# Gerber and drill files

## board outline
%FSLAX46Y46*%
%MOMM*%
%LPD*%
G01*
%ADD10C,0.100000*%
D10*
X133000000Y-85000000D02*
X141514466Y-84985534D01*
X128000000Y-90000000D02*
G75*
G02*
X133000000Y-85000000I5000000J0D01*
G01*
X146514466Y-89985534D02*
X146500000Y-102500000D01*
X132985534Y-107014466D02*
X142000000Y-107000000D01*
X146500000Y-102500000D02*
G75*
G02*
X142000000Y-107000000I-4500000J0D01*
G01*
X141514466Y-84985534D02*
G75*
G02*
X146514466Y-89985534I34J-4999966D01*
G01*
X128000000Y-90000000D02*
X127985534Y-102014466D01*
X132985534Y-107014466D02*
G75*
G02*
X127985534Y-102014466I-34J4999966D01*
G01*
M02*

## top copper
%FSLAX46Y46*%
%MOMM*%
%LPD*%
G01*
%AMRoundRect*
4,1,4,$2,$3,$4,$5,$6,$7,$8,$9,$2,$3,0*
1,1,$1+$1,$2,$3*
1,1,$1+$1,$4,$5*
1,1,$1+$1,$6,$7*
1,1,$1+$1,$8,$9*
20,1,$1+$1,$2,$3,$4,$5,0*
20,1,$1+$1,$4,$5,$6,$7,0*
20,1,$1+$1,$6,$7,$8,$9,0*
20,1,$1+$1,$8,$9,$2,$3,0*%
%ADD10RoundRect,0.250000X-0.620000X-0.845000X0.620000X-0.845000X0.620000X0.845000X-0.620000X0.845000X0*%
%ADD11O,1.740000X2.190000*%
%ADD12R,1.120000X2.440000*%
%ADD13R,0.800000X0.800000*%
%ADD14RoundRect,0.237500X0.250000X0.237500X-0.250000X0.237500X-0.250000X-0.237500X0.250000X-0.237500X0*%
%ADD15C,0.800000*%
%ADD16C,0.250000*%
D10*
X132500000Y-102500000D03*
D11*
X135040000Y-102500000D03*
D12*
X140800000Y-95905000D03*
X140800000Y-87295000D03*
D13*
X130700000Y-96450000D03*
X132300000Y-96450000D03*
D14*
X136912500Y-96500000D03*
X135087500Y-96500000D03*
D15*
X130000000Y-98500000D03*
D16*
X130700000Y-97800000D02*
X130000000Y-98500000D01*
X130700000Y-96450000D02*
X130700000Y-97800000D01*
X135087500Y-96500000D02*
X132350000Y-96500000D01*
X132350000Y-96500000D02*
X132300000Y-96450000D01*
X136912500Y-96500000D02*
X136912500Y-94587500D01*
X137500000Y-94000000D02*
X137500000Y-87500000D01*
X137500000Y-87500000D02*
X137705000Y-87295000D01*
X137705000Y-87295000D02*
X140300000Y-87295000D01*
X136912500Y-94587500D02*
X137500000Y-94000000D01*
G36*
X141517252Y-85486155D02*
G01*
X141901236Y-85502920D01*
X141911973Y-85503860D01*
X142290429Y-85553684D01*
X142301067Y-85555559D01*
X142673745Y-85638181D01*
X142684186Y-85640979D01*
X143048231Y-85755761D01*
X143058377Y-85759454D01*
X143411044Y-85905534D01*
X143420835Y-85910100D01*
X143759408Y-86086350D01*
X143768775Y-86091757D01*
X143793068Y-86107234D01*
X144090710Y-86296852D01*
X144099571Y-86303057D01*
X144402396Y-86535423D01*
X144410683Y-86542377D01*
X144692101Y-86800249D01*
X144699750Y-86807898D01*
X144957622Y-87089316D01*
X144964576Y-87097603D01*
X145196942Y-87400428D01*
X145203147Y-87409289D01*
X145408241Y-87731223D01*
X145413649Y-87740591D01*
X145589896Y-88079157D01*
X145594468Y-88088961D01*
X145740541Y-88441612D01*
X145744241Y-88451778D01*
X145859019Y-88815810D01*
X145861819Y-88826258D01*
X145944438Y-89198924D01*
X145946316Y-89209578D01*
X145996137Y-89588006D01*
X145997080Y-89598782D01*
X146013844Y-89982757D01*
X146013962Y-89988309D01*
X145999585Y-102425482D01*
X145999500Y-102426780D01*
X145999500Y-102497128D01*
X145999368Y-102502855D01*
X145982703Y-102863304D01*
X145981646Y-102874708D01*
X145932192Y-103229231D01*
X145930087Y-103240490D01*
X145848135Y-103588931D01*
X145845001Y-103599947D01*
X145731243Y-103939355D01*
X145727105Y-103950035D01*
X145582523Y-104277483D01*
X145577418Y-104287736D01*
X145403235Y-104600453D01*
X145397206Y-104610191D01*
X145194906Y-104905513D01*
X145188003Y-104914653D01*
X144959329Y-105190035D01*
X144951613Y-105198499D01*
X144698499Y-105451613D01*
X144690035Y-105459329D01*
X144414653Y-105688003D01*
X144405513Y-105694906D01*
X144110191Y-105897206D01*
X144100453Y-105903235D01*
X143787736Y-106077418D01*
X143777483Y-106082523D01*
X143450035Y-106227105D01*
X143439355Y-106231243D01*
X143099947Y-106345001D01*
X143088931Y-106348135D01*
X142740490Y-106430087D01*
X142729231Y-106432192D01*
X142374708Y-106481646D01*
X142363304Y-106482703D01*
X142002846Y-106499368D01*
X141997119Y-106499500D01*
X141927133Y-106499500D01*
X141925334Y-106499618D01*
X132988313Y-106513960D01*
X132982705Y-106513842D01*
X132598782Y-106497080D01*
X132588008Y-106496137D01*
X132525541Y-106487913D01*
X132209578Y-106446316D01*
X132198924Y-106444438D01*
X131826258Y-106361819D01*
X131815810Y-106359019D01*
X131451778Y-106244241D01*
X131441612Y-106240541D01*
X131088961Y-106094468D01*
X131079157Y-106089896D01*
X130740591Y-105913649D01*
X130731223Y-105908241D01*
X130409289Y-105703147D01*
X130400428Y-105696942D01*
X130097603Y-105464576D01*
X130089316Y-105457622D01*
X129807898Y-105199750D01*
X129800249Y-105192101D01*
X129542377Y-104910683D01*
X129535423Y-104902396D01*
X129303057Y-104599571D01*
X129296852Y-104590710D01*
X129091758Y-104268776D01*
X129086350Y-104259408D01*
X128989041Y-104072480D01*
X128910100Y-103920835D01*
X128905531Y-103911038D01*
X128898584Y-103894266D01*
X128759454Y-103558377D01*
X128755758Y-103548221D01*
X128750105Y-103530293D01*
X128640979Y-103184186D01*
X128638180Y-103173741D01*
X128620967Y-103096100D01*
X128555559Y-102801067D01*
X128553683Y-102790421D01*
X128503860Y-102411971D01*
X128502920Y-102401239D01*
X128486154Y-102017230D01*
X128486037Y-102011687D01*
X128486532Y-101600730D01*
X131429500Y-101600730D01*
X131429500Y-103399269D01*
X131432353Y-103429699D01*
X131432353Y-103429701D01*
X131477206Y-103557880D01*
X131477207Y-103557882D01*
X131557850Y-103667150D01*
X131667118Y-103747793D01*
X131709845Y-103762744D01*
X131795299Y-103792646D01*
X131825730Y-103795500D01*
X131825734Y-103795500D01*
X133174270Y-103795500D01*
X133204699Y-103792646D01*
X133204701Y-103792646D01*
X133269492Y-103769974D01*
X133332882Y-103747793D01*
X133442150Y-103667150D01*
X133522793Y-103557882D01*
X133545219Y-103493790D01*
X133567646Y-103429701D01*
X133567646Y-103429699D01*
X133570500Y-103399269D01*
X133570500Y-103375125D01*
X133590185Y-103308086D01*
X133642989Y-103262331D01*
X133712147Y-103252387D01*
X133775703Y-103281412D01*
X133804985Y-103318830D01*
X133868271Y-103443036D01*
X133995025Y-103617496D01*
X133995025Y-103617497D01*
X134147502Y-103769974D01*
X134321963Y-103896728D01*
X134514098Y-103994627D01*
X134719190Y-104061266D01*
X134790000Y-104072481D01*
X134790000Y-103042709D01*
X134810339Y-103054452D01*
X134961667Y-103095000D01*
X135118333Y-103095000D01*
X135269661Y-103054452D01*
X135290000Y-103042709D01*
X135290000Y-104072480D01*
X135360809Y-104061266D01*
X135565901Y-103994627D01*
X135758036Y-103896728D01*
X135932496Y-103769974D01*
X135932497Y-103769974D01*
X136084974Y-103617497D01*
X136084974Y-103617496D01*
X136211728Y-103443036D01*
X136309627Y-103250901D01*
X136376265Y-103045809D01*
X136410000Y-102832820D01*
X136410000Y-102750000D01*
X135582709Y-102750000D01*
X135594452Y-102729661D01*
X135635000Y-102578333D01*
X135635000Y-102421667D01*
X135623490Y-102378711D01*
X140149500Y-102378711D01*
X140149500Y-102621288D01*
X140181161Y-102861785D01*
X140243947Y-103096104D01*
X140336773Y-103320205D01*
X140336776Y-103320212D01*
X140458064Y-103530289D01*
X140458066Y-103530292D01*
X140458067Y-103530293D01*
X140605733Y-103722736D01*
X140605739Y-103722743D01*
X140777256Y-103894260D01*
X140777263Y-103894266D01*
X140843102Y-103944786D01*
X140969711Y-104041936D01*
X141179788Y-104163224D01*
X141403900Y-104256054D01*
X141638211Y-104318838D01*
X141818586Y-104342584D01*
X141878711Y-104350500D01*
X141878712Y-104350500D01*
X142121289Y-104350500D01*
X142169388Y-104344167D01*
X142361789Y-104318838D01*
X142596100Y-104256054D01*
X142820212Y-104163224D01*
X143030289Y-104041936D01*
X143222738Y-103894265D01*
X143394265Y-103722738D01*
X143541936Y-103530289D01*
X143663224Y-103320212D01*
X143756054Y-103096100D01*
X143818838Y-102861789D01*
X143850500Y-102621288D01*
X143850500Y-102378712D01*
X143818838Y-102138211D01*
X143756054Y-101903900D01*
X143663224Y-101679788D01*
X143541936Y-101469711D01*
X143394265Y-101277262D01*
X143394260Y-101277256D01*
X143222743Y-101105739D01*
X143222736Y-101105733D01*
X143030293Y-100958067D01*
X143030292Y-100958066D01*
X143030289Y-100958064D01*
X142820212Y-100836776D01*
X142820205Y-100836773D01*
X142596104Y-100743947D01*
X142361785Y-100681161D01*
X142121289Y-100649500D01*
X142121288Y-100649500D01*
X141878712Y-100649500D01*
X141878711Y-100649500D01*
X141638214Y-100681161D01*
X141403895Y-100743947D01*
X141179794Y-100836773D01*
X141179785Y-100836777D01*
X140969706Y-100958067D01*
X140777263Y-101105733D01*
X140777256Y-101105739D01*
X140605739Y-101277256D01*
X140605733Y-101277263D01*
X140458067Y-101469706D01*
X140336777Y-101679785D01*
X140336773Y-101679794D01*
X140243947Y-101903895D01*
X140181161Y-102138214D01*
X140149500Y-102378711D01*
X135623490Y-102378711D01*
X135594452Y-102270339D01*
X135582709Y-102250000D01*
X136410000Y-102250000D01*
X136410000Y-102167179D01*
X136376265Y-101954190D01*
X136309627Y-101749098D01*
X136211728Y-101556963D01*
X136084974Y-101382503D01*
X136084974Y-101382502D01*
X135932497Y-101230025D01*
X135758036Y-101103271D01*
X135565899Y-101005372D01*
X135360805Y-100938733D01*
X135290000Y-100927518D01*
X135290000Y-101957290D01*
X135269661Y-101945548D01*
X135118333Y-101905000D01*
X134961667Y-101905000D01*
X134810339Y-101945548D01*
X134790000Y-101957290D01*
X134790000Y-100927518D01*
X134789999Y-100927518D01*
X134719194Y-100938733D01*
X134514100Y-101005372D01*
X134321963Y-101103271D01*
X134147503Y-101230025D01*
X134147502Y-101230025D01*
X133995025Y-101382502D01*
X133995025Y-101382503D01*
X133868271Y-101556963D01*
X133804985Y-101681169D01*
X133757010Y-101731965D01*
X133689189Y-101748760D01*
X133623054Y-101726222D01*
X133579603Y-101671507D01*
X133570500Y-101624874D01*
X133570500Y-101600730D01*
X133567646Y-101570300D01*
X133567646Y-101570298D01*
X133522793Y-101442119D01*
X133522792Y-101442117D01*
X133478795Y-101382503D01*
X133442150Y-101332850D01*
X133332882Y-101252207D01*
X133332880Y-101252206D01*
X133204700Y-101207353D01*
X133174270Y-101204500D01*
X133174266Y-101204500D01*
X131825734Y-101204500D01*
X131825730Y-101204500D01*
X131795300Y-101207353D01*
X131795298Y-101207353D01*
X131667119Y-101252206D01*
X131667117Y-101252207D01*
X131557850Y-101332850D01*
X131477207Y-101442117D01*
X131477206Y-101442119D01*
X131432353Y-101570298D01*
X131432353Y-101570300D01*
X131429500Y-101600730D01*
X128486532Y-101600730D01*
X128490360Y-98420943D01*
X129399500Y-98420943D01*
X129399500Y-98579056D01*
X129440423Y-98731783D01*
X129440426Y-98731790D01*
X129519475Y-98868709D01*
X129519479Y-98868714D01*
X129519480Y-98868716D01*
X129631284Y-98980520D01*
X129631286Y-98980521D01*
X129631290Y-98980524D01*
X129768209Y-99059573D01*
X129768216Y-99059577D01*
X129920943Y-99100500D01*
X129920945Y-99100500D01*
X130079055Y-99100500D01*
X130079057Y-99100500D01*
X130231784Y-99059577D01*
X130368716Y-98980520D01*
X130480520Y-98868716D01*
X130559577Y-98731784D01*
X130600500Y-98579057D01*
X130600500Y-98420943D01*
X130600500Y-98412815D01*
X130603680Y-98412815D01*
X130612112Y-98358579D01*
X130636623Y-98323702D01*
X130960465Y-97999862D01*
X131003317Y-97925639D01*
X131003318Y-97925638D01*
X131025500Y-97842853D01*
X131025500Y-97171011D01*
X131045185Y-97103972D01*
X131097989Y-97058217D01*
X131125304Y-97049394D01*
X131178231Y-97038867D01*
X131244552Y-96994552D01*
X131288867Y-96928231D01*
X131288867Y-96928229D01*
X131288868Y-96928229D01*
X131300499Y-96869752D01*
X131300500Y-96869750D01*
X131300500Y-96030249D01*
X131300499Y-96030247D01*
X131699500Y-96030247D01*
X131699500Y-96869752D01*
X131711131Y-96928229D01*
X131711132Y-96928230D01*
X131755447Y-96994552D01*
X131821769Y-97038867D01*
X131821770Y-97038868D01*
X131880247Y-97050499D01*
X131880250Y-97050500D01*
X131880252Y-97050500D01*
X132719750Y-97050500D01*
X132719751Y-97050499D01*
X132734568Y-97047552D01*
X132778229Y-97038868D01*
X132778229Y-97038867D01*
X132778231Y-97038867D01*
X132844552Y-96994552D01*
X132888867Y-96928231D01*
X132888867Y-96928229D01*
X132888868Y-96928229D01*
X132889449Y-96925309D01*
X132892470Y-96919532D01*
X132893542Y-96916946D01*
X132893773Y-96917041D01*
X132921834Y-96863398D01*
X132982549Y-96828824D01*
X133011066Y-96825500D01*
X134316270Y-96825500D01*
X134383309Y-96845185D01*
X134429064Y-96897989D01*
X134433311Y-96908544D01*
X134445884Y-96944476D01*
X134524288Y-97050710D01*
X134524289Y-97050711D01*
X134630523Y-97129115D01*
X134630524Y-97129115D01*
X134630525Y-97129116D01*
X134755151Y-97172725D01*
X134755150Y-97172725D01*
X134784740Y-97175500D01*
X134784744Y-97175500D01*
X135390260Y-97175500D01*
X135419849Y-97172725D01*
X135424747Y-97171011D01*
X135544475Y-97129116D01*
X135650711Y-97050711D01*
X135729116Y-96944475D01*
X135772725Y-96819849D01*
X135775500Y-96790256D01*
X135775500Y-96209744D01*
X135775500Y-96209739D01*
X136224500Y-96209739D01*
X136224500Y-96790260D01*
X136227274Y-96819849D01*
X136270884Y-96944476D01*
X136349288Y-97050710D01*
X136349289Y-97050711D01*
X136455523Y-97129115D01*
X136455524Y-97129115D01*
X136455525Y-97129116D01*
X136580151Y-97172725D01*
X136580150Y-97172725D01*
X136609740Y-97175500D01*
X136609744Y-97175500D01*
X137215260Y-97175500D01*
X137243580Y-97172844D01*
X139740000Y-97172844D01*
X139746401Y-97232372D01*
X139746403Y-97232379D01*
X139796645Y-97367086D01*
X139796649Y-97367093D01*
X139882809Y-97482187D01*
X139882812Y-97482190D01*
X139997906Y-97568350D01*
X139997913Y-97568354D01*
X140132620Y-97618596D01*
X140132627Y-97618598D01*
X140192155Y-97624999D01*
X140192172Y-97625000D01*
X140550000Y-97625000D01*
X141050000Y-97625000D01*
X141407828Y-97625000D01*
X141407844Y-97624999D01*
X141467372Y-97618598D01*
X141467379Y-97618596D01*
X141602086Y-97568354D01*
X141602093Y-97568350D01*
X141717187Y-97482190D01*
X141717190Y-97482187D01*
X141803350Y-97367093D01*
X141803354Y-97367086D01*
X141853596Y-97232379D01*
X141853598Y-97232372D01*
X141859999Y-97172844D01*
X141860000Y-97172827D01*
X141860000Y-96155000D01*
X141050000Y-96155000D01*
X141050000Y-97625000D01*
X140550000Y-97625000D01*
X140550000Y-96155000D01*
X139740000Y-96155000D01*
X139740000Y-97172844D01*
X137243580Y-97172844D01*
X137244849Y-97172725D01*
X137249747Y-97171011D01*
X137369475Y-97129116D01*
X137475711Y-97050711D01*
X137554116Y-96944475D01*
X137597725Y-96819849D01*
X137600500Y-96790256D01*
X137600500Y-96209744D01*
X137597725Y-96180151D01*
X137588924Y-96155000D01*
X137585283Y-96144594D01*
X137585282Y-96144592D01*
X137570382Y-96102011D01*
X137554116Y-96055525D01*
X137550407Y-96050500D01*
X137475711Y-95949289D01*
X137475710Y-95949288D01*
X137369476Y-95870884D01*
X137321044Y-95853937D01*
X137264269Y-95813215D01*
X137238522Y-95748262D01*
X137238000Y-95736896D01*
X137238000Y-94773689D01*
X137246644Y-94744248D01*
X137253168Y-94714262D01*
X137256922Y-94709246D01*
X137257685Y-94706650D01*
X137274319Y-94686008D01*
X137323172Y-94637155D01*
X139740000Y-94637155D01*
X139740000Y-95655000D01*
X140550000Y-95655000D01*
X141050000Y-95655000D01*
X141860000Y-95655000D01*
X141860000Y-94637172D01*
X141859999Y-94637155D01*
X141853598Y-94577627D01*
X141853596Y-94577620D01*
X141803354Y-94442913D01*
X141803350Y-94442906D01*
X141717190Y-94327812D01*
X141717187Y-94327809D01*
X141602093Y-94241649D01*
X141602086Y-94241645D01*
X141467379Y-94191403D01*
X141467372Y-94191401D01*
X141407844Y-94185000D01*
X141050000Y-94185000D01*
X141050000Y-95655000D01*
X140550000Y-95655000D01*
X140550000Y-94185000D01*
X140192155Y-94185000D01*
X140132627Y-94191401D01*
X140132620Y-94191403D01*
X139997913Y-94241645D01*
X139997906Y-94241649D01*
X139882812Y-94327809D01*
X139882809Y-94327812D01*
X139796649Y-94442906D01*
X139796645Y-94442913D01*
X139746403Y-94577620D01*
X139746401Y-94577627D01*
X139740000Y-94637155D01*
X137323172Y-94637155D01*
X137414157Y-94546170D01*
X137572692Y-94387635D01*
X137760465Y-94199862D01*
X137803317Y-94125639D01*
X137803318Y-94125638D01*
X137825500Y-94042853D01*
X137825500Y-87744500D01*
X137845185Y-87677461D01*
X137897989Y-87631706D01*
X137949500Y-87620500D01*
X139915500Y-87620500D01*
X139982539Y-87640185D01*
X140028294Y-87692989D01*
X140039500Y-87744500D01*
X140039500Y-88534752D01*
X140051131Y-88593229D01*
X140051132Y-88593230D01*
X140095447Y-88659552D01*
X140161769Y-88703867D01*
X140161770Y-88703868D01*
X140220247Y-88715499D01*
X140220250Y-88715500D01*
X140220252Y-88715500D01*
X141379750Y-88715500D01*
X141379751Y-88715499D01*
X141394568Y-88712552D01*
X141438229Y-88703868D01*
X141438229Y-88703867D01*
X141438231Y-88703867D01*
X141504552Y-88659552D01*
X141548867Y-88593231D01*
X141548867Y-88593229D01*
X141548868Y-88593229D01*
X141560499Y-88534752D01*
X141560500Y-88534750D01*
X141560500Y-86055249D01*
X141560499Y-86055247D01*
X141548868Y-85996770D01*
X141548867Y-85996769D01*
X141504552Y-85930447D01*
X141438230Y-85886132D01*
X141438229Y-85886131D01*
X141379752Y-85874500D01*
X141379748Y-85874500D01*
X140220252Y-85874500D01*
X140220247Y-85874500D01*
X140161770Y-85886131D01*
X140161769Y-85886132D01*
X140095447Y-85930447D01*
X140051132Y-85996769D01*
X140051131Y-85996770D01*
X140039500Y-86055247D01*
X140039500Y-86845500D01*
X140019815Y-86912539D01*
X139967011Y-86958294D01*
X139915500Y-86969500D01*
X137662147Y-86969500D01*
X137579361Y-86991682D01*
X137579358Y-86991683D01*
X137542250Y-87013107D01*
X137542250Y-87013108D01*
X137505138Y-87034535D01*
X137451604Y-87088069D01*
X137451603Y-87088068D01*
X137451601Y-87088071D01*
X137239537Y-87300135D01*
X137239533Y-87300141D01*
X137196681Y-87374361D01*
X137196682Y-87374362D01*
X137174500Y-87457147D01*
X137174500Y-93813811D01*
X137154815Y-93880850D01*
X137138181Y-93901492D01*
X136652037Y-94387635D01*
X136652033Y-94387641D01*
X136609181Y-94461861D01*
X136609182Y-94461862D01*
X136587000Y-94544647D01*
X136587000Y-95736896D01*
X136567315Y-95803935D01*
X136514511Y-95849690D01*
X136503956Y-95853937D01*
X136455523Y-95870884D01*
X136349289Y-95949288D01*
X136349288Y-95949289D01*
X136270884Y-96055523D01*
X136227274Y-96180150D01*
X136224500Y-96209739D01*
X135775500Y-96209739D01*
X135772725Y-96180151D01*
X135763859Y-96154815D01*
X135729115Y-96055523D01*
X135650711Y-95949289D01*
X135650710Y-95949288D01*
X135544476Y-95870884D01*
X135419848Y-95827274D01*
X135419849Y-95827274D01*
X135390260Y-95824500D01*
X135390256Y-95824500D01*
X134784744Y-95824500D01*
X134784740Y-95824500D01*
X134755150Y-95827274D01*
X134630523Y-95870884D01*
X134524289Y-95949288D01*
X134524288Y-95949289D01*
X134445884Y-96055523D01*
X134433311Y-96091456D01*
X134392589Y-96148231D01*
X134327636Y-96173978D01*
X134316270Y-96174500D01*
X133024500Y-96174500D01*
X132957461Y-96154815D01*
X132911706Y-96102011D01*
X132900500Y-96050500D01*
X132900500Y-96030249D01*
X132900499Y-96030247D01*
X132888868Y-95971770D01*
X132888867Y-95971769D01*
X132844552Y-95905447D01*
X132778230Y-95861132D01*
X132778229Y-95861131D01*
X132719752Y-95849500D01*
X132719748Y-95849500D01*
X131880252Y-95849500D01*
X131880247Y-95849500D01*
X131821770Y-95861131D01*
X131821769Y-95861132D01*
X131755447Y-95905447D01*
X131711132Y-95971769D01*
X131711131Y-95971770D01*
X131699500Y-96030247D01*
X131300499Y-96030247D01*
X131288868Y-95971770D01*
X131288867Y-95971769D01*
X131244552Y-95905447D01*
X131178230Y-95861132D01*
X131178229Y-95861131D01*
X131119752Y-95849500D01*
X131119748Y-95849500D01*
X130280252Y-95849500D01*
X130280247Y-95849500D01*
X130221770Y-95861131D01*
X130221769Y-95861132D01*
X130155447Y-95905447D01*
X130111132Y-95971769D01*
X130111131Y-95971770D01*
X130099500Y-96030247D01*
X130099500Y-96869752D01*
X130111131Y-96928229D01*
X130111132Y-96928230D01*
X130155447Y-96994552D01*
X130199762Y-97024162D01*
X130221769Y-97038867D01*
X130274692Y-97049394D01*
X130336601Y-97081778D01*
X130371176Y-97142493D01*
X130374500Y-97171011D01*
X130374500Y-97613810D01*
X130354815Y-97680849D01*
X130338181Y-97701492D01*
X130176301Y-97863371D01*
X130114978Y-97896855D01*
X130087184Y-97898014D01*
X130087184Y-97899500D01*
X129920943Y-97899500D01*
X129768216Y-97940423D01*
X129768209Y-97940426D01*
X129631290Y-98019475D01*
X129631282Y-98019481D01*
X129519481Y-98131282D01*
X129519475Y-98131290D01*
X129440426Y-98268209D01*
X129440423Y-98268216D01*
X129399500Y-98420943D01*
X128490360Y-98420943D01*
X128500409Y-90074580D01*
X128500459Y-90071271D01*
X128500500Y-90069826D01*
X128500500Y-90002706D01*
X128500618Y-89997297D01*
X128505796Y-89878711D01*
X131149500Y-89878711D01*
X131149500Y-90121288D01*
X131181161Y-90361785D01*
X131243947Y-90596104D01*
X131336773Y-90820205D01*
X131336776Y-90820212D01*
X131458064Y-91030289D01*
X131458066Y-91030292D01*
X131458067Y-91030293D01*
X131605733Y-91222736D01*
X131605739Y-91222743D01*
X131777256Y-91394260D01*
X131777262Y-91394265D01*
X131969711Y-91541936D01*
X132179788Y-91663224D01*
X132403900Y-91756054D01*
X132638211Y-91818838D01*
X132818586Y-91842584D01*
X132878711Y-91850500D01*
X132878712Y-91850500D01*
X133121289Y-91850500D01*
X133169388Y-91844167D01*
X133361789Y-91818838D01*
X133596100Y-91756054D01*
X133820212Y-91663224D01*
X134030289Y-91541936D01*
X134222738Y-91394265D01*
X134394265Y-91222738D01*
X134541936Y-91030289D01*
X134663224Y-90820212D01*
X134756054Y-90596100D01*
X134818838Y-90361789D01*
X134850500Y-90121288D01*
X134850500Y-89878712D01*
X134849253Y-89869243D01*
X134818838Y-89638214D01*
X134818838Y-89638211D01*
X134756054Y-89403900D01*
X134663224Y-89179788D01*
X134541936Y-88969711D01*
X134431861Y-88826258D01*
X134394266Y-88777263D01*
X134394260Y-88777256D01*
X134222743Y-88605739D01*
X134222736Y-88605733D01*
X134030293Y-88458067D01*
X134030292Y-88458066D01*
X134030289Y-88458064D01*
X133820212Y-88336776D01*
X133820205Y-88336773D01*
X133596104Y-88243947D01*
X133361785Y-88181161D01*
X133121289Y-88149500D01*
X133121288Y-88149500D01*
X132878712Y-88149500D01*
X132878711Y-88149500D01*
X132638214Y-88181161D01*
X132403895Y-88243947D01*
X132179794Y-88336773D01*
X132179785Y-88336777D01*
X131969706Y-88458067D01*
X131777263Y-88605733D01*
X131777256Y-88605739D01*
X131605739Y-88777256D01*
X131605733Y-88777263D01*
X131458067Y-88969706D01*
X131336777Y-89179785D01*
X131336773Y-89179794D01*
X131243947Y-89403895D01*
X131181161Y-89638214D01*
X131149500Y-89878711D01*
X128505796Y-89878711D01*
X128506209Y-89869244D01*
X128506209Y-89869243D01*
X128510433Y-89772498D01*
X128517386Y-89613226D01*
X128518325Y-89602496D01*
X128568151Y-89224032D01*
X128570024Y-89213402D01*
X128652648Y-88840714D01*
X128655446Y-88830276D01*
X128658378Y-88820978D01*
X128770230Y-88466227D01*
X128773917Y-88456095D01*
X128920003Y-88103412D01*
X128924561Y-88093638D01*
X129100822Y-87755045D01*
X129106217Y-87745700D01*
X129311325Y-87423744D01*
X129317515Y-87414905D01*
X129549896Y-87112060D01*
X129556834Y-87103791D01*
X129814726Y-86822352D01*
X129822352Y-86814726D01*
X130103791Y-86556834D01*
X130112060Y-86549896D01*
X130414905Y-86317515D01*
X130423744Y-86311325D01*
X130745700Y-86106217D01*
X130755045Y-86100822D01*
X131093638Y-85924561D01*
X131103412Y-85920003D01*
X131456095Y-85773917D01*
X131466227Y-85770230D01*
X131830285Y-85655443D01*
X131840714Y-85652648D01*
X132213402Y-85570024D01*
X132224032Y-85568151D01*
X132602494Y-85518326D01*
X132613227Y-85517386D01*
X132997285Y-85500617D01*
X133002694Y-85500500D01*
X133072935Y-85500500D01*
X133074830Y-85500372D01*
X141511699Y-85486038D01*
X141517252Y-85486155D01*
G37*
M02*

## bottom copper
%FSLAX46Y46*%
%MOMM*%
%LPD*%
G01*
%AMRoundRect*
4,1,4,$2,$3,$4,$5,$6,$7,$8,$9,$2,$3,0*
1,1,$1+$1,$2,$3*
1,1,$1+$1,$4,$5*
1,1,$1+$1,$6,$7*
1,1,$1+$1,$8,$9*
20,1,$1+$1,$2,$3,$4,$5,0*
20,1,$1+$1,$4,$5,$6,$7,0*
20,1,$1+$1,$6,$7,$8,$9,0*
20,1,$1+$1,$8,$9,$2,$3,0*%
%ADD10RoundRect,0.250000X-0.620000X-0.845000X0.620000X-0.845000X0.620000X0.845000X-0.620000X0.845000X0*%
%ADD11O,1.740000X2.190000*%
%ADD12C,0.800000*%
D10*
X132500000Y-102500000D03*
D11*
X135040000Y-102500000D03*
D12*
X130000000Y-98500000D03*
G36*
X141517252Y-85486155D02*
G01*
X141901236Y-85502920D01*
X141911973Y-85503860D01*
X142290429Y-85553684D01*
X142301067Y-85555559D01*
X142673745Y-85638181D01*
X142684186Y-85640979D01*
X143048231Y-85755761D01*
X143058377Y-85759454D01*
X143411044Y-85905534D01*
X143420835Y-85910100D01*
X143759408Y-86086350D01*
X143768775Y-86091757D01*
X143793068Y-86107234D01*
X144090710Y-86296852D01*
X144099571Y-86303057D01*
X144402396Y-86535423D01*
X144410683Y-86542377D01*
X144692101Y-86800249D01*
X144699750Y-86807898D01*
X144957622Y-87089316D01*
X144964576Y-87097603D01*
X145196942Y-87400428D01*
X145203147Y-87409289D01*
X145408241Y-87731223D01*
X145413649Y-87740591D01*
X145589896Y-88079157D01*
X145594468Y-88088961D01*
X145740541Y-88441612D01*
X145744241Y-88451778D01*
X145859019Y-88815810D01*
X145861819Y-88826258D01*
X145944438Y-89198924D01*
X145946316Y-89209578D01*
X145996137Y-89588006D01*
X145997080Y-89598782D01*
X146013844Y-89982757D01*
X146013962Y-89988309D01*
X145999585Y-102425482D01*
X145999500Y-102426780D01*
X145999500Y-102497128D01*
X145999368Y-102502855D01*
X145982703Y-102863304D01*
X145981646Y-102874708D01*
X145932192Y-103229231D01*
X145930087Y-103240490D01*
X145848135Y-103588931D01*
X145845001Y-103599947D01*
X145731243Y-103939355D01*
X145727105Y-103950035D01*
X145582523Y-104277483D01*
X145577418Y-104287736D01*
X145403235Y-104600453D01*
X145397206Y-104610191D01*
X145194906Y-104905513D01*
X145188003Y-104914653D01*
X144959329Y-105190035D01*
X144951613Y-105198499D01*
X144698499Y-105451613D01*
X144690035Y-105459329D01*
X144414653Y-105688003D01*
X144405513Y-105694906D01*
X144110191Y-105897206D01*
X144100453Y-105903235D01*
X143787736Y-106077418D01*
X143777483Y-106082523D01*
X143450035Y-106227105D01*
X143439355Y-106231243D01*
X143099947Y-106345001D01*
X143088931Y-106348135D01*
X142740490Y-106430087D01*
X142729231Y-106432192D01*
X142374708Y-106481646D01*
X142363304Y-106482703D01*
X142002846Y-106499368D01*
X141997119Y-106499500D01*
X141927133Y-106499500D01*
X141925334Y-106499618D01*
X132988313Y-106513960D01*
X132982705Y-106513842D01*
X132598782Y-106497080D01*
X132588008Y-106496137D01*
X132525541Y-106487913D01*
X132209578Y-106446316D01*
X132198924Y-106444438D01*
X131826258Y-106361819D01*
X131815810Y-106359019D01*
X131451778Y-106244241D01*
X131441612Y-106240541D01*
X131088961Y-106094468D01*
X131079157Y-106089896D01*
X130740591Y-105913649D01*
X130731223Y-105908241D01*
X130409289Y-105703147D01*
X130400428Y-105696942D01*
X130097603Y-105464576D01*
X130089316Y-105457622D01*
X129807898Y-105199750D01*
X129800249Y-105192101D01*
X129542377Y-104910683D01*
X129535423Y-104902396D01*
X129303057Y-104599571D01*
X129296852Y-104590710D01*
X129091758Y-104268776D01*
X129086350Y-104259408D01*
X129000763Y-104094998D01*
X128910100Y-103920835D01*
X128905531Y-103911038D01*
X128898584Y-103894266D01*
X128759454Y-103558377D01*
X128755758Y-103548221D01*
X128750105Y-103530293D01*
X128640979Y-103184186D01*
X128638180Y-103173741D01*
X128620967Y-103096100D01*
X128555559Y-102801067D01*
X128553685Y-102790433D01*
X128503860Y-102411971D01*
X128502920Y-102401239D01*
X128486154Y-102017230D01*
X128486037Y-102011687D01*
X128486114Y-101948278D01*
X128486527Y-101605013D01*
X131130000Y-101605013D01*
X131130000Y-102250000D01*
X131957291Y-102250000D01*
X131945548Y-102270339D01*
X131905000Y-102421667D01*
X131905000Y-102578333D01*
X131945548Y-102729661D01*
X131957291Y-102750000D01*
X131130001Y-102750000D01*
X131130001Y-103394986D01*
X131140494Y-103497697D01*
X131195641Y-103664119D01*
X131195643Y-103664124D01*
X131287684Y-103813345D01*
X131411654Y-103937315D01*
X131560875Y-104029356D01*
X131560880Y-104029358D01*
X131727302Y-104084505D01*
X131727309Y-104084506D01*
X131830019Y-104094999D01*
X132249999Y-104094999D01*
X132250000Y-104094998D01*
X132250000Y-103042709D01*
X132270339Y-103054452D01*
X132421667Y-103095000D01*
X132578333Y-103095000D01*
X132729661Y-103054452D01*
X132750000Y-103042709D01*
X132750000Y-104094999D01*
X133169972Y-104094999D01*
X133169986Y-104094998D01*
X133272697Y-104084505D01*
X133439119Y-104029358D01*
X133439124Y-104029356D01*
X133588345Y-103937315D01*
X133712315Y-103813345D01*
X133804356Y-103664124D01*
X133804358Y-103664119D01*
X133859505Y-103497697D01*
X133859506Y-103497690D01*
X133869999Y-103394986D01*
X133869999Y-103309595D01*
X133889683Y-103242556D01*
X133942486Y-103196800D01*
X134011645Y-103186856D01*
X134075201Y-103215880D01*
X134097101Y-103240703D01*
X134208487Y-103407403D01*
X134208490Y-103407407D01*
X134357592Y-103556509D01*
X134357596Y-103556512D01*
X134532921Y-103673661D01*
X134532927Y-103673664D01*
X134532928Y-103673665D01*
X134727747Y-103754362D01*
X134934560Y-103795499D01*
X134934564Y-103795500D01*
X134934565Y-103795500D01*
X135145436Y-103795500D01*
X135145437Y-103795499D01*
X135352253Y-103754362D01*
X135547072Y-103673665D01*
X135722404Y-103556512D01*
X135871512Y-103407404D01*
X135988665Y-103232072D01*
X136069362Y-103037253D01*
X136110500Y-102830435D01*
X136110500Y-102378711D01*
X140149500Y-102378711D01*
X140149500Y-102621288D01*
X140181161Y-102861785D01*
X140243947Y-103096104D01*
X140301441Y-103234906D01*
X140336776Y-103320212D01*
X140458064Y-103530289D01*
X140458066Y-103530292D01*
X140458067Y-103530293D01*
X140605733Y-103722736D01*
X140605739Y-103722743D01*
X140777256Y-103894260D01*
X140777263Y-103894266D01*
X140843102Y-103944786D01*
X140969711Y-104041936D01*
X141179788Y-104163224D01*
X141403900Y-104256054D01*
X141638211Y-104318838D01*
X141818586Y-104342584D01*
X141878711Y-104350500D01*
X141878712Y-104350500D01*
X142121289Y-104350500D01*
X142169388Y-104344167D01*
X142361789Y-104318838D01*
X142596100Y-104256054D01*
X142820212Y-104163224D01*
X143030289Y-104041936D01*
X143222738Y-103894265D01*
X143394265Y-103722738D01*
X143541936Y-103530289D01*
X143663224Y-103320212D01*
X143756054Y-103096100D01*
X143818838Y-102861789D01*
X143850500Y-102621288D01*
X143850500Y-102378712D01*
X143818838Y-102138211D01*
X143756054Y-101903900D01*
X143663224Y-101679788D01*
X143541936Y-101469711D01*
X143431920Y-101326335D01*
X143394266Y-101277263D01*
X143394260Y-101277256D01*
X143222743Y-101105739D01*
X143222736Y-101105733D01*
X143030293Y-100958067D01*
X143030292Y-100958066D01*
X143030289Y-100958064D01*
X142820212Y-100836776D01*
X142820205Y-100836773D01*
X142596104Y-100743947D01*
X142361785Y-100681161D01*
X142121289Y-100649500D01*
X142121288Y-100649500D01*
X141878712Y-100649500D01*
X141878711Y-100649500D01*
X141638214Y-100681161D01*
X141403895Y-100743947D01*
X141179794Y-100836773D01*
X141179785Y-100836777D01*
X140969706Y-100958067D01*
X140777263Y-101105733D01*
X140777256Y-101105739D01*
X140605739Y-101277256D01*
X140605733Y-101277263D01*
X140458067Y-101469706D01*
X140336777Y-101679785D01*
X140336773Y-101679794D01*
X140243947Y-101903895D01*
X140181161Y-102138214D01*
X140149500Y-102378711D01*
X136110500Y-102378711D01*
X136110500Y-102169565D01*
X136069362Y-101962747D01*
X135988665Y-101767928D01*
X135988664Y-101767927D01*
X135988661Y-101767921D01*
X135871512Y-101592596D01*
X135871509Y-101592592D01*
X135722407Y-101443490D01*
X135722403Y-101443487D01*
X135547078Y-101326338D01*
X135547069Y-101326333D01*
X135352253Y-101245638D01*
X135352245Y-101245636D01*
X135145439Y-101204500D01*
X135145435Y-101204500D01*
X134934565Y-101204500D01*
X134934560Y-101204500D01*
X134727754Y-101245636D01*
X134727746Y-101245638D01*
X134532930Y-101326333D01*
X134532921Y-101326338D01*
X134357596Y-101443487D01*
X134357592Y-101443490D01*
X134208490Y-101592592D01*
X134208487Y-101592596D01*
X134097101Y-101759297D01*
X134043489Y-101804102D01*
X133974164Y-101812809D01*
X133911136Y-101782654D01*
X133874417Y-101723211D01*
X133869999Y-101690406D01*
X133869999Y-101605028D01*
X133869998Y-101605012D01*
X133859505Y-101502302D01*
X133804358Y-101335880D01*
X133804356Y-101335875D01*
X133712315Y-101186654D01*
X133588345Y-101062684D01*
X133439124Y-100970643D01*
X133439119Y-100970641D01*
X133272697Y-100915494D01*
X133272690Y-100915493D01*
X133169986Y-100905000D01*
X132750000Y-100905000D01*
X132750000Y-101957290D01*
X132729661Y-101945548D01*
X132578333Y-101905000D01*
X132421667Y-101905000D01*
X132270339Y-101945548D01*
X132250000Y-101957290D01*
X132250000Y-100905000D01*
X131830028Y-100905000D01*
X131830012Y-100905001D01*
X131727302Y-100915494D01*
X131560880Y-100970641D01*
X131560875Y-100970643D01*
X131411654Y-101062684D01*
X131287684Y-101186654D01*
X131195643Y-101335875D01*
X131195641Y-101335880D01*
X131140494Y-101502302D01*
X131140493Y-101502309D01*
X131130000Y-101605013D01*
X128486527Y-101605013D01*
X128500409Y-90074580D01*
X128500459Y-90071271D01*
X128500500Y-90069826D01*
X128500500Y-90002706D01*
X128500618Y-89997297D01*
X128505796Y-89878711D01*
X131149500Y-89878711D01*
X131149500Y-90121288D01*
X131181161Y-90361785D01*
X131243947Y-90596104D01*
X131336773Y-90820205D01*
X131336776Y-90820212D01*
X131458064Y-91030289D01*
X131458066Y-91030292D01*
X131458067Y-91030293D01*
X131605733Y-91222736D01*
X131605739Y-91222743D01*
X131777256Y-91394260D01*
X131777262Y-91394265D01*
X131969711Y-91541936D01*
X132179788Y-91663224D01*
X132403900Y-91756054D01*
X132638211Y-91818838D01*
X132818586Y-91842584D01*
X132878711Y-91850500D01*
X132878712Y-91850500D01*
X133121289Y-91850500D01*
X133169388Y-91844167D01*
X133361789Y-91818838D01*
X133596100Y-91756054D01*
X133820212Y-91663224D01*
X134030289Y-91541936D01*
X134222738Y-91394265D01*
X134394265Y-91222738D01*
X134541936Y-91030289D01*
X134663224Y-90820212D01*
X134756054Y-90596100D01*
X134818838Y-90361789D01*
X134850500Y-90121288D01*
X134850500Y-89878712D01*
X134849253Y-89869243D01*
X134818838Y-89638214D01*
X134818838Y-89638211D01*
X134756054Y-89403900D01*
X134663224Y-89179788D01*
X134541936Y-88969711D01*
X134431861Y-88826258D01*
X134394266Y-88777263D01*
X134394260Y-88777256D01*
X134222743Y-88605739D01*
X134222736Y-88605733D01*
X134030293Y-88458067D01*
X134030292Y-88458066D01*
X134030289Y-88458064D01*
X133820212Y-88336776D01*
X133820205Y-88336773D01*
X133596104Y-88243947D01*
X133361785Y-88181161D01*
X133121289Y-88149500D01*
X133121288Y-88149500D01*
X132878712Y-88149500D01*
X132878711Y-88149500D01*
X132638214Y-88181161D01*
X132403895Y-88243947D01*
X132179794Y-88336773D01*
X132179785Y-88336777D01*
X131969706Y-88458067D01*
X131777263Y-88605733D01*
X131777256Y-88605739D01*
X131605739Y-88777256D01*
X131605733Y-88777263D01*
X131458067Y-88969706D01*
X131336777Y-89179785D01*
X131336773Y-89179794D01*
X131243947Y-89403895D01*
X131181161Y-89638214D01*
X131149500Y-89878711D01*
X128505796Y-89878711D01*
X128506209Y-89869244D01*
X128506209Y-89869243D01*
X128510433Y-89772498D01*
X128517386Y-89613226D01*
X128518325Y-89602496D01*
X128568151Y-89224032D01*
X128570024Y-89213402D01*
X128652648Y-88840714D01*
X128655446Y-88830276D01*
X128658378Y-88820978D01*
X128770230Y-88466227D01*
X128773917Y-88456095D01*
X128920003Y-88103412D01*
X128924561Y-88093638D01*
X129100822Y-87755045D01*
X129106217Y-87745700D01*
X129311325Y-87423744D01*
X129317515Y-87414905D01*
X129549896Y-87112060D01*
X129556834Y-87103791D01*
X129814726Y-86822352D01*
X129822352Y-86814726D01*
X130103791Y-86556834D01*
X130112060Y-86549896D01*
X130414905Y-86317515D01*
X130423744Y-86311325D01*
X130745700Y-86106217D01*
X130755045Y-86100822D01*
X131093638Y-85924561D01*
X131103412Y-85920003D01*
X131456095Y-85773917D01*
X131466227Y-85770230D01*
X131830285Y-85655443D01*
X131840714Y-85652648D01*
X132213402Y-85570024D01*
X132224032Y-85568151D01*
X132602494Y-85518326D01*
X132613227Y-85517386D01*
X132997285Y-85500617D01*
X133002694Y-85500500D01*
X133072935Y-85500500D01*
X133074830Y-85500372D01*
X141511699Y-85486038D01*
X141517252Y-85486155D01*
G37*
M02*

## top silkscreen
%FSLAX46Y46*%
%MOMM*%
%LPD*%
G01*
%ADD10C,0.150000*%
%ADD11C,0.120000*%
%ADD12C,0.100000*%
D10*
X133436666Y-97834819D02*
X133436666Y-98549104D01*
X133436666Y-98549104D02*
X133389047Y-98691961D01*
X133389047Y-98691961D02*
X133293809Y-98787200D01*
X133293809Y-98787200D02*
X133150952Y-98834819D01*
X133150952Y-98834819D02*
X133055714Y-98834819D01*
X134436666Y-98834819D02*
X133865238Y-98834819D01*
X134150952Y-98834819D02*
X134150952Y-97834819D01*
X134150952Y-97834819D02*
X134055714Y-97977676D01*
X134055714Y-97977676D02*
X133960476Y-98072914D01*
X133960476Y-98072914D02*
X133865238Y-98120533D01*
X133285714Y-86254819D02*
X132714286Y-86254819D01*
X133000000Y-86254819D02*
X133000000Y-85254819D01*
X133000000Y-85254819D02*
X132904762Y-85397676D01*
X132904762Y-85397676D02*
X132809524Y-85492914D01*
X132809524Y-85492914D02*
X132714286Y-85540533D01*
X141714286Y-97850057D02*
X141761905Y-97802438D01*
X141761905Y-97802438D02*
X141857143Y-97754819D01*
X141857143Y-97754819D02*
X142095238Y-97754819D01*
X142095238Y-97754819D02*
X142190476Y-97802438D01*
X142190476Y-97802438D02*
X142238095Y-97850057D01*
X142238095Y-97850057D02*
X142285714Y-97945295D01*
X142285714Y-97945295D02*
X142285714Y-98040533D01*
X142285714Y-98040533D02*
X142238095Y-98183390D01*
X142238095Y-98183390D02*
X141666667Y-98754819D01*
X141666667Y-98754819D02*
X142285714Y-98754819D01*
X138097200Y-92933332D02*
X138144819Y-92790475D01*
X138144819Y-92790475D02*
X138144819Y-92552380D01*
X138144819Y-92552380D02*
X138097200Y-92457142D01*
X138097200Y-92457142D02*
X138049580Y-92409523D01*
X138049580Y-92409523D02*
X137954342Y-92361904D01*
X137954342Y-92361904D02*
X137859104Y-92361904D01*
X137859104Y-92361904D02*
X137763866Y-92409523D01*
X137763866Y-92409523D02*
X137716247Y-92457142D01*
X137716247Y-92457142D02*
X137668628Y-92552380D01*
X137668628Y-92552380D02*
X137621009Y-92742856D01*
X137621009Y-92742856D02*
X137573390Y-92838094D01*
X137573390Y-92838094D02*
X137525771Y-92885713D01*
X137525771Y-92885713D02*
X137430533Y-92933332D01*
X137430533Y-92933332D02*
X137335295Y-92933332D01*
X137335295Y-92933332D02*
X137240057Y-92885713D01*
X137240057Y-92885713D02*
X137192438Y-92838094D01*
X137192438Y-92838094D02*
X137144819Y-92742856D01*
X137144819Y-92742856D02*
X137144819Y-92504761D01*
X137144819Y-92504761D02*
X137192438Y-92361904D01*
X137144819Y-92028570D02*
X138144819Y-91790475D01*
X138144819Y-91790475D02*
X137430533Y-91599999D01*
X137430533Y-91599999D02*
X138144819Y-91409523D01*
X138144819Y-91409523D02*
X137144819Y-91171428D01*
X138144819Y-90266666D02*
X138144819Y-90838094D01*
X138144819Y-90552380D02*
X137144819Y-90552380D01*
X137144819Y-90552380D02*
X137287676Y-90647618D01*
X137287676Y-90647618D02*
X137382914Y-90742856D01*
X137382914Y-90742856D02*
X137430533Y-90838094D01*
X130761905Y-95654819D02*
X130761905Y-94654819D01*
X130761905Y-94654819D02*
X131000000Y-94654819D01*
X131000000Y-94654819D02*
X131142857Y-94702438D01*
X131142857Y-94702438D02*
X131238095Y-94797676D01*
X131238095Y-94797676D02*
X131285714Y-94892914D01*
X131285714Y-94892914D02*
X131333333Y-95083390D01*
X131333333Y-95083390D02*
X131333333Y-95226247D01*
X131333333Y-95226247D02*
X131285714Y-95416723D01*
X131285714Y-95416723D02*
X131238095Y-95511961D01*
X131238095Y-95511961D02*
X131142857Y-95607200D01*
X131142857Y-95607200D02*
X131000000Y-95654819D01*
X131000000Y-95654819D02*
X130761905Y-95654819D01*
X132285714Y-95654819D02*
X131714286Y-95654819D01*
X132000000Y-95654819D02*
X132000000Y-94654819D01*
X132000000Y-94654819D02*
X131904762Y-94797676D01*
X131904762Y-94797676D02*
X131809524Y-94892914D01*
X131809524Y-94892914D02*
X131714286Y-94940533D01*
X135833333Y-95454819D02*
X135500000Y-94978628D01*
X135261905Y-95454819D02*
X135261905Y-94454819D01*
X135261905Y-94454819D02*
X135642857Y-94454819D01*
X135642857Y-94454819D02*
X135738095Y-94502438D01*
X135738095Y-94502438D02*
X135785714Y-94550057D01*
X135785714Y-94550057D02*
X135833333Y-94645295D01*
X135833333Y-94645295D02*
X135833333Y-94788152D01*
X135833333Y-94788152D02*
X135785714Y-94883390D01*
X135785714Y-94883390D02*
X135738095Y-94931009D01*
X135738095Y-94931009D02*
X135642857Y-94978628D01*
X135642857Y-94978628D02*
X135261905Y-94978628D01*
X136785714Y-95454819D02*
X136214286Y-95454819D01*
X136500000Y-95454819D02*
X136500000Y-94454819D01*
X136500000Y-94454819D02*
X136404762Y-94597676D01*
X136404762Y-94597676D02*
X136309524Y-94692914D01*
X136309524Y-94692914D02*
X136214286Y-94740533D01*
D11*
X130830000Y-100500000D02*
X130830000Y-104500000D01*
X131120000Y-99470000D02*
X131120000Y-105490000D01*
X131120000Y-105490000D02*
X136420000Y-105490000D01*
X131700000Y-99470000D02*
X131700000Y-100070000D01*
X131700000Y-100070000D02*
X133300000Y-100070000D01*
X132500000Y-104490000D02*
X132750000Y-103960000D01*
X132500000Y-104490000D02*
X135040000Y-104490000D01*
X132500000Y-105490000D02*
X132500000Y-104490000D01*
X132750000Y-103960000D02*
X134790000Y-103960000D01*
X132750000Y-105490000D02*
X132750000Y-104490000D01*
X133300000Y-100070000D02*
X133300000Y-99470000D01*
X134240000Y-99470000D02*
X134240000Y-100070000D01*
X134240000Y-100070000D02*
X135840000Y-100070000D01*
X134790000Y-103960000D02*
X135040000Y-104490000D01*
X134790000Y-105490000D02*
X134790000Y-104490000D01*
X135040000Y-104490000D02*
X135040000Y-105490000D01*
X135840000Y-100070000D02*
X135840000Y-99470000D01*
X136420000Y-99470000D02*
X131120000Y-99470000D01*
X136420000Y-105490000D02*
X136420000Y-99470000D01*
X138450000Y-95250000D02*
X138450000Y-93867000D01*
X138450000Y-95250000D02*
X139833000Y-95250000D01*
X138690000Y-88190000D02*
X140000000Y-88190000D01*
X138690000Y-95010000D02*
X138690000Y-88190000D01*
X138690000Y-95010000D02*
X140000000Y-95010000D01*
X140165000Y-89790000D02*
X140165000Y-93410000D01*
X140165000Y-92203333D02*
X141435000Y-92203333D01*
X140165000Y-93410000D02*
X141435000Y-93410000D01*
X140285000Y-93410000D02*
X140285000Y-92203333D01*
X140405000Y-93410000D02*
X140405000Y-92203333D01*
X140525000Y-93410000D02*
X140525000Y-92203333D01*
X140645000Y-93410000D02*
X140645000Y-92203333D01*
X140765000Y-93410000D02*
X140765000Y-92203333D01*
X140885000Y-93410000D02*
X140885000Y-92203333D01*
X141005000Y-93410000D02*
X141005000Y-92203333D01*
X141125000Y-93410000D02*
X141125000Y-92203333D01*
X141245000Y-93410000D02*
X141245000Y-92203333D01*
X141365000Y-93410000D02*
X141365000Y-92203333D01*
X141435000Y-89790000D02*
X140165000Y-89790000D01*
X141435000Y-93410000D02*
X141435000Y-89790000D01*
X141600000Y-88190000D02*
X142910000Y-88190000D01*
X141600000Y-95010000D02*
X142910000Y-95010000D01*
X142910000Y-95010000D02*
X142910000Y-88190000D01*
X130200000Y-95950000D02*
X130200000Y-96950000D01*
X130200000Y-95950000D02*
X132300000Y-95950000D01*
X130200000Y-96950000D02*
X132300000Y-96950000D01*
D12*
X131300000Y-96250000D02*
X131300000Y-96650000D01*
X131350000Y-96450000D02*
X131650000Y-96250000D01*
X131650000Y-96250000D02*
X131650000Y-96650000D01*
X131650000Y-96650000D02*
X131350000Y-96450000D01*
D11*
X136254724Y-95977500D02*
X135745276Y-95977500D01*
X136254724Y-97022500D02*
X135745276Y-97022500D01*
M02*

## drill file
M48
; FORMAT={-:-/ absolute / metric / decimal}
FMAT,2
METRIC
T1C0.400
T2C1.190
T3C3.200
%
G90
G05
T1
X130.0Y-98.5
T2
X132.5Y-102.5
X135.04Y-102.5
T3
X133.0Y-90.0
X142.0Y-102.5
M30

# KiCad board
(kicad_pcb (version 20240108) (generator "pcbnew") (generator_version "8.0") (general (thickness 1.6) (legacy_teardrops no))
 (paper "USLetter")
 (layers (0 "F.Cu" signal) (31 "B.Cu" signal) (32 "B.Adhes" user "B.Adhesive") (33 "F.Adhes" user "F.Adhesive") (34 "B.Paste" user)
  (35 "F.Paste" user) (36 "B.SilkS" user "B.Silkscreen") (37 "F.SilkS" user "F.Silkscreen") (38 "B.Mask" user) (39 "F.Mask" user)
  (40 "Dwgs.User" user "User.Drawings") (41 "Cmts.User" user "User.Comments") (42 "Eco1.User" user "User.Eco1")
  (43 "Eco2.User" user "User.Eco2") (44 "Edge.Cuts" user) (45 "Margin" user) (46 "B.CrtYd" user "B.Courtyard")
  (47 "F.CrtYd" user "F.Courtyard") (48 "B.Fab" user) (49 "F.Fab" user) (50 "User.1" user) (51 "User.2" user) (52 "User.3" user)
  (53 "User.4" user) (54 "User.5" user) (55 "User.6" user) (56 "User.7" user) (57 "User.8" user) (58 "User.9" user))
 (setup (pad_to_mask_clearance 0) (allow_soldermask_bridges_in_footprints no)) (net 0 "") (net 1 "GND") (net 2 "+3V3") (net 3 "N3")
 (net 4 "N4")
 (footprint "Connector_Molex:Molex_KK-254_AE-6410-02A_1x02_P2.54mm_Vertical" (layer "F.Cu") (at 132.5 102.5)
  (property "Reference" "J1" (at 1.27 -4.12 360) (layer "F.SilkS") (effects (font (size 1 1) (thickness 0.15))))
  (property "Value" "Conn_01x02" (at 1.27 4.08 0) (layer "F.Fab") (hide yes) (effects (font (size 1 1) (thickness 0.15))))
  (fp_line (start -1.67 -2) (end -1.67 2) (stroke (width 0.12) (type solid)) (layer "F.SilkS"))
  (fp_line (start -1.38 -3.03) (end -1.38 2.99) (stroke (width 0.12) (type solid)) (layer "F.SilkS"))
  (fp_line (start -1.38 2.99) (end 3.92 2.99) (stroke (width 0.12) (type solid)) (layer "F.SilkS"))
  (fp_line (start -0.8 -3.03) (end -0.8 -2.43) (stroke (width 0.12) (type solid)) (layer "F.SilkS"))
  (fp_line (start -0.8 -2.43) (end 0.8 -2.43) (stroke (width 0.12) (type solid)) (layer "F.SilkS"))
  (fp_line (start 0 1.99) (end 0.25 1.46) (stroke (width 0.12) (type solid)) (layer "F.SilkS"))
  (fp_line (start 0 1.99) (end 2.54 1.99) (stroke (width 0.12) (type solid)) (layer "F.SilkS"))
  (fp_line (start 0 2.99) (end 0 1.99) (stroke (width 0.12) (type solid)) (layer "F.SilkS"))
  (fp_line (start 0.25 1.46) (end 2.29 1.46) (stroke (width 0.12) (type solid)) (layer "F.SilkS"))
  (fp_line (start 0.25 2.99) (end 0.25 1.99) (stroke (width 0.12) (type solid)) (layer "F.SilkS"))
  (fp_line (start 0.8 -2.43) (end 0.8 -3.03) (stroke (width 0.12) (type solid)) (layer "F.SilkS"))
  (fp_line (start 1.74 -3.03) (end 1.74 -2.43) (stroke (width 0.12) (type solid)) (layer "F.SilkS"))
  (fp_line (start 1.74 -2.43) (end 3.34 -2.43) (stroke (width 0.12) (type solid)) (layer "F.SilkS"))
  (fp_line (start 2.29 1.46) (end 2.54 1.99) (stroke (width 0.12) (type solid)) (layer "F.SilkS"))
  (fp_line (start 2.29 2.99) (end 2.29 1.99) (stroke (width 0.12) (type solid)) (layer "F.SilkS"))
  (fp_line (start 2.54 1.99) (end 2.54 2.99) (stroke (width 0.12) (type solid)) (layer "F.SilkS"))
  (fp_line (start 3.34 -2.43) (end 3.34 -3.03) (stroke (width 0.12) (type solid)) (layer "F.SilkS"))
  (fp_line (start 3.92 -3.03) (end -1.38 -3.03) (stroke (width 0.12) (type solid)) (layer "F.SilkS"))
  (fp_line (start 3.92 2.99) (end 3.92 -3.03) (stroke (width 0.12) (type solid)) (layer "F.SilkS"))
  (pad "1" thru_hole roundrect (at 0 0) (size 1.74 2.19) (drill 1.19) (layers "*.Cu" "*.Mask") (remove_unused_layers no)
   (roundrect_rratio 0.143678) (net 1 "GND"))
  (pad "2" thru_hole oval (at 2.54 0) (size 1.74 2.19) (drill 1.19) (layers "*.Cu" "*.Mask") (remove_unused_layers no) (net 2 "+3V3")))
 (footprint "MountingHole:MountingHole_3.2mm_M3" (layer "F.Cu") (at 133 90)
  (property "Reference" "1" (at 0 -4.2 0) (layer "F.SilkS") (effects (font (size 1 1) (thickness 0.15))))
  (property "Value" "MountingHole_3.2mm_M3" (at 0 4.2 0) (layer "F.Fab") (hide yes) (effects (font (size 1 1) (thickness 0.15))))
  (pad "" np_thru_hole circle (at 0 0) (size 3.2 3.2) (drill 3.2) (layers "*.Cu" "*.Mask")))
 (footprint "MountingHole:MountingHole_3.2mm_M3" (layer "F.Cu") (at 142 102.5)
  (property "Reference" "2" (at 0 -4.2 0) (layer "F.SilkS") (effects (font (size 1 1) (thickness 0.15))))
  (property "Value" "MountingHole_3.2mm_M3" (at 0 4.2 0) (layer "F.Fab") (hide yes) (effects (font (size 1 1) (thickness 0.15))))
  (pad "" np_thru_hole circle (at 0 0) (size 3.2 3.2) (drill 3.2) (layers "F&B.Cu" "*.Mask")))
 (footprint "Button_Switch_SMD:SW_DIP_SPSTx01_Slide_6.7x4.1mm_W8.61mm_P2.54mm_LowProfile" (layer "F.Cu") (at 140.8 91.6 90)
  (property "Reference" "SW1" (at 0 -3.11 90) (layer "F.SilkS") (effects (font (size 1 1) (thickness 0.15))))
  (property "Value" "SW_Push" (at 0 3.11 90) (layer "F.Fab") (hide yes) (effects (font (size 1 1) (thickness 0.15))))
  (fp_line (start -3.65 -2.35) (end -2.267 -2.35) (stroke (width 0.12) (type solid)) (layer "F.SilkS"))
  (fp_line (start -3.65 -2.35) (end -3.65 -0.967) (stroke (width 0.12) (type solid)) (layer "F.SilkS"))
  (fp_line (start 3.41 -2.11) (end 3.41 -0.8) (stroke (width 0.12) (type solid)) (layer "F.SilkS"))
  (fp_line (start -3.41 -2.11) (end 3.41 -2.11) (stroke (width 0.12) (type solid)) (layer "F.SilkS"))
  (fp_line (start -3.41 -2.11) (end -3.41 -0.8) (stroke (width 0.12) (type solid)) (layer "F.SilkS"))
  (fp_line (start 1.81 -0.635) (end -1.81 -0.635) (stroke (width 0.12) (type solid)) (layer "F.SilkS"))
  (fp_line (start -0.603333 -0.635) (end -0.603333 0.635) (stroke (width 0.12) (type solid)) (layer "F.SilkS"))
  (fp_line (start -1.81 -0.635) (end -1.81 0.635) (stroke (width 0.12) (type solid)) (layer "F.SilkS"))
  (fp_line (start -1.81 -0.515) (end -0.603333 -0.515) (stroke (width 0.12) (type solid)) (layer "F.SilkS"))
  (fp_line (start -1.81 -0.395) (end -0.603333 -0.395) (stroke (width 0.12) (type solid)) (layer "F.SilkS"))
  (fp_line (start -1.81 -0.275) (end -0.603333 -0.275) (stroke (width 0.12) (type solid)) (layer "F.SilkS"))
  (fp_line (start -1.81 -0.155) (end -0.603333 -0.155) (stroke (width 0.12) (type solid)) (layer "F.SilkS"))
  (fp_line (start -1.81 -0.035) (end -0.603333 -0.035) (stroke (width 0.12) (type solid)) (layer "F.SilkS"))
  (fp_line (start -1.81 0.085) (end -0.603333 0.085) (stroke (width 0.12) (type solid)) (layer "F.SilkS"))
  (fp_line (start -1.81 0.205) (end -0.603333 0.205) (stroke (width 0.12) (type solid)) (layer "F.SilkS"))
  (fp_line (start -1.81 0.325) (end -0.603333 0.325) (stroke (width 0.12) (type solid)) (layer "F.SilkS"))
  (fp_line (start -1.81 0.445) (end -0.603333 0.445) (stroke (width 0.12) (type solid)) (layer "F.SilkS"))
  (fp_line (start -1.81 0.565) (end -0.603333 0.565) (stroke (width 0.12) (type solid)) (layer "F.SilkS"))
  (fp_line (start 1.81 0.635) (end 1.81 -0.635) (stroke (width 0.12) (type solid)) (layer "F.SilkS"))
  (fp_line (start -1.81 0.635) (end 1.81 0.635) (stroke (width 0.12) (type solid)) (layer "F.SilkS"))
  (fp_line (start 3.41 0.8) (end 3.41 2.11) (stroke (width 0.12) (type solid)) (layer "F.SilkS"))
  (fp_line (start -3.41 0.8) (end -3.41 2.11) (stroke (width 0.12) (type solid)) (layer "F.SilkS"))
  (fp_line (start -3.41 2.11) (end 3.41 2.11) (stroke (width 0.12) (type solid)) (layer "F.SilkS"))
  (pad "1" smd rect (at -4.305 0 90) (size 2.44 1.12) (layers "F.Cu" "F.Paste" "F.Mask") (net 2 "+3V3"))
  (pad "2" smd rect (at 4.305 0 90) (size 2.44 1.12) (layers "F.Cu" "F.Paste" "F.Mask") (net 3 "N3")))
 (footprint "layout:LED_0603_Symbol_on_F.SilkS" (layer "F.Cu") (at 131.5 96.45)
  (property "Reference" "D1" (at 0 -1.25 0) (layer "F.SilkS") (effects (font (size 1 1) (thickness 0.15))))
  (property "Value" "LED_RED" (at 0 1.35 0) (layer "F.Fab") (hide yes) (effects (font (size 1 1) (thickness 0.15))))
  (fp_line (start -1.3 -0.5) (end -1.3 0.5) (stroke (width 0.12) (type solid)) (layer "F.SilkS"))
  (fp_line (start -1.3 -0.5) (end 0.8 -0.5) (stroke (width 0.12) (type solid)) (layer "F.SilkS"))
  (fp_line (start -1.3 0.5) (end 0.8 0.5) (stroke (width 0.12) (type solid)) (layer "F.SilkS"))
  (fp_line (start -0.2 -0.2) (end -0.2 0.2) (stroke (width 0.1) (type solid)) (layer "F.SilkS"))
  (fp_line (start -0.15 0) (end 0.15 -0.2) (stroke (width 0.1) (type solid)) (layer "F.SilkS"))
  (fp_line (start 0.15 -0.2) (end 0.15 0.2) (stroke (width 0.1) (type solid)) (layer "F.SilkS"))
  (fp_line (start 0.15 0.2) (end -0.15 0) (stroke (width 0.1) (type solid)) (layer "F.SilkS"))
  (pad "1" smd rect (at -0.8 0 180) (size 0.8 0.8) (layers "F.Cu" "F.Paste" "F.Mask") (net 1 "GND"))
  (pad "2" smd rect (at 0.8 0 180) (size 0.8 0.8) (layers "F.Cu" "F.Paste" "F.Mask") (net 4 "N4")))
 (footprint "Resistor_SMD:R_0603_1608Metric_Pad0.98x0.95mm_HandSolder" (layer "F.Cu") (at 136 96.5 180)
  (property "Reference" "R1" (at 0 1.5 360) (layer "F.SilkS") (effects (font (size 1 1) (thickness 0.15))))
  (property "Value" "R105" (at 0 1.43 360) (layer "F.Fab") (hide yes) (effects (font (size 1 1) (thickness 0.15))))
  (fp_line (start -0.254724 0.5225) (end 0.254724 0.5225) (stroke (width 0.12) (type solid)) (layer "F.SilkS"))
  (fp_line (start -0.254724 -0.5225) (end 0.254724 -0.5225) (stroke (width 0.12) (type solid)) (layer "F.SilkS"))
  (pad "1" smd roundrect (at -0.9125 0 180) (size 0.975 0.95) (layers "F.Cu" "F.Paste" "F.Mask") (roundrect_rratio 0.25) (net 3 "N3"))
  (pad "2" smd roundrect (at 0.9125 0 180) (size 0.975 0.95) (layers "F.Cu" "F.Paste" "F.Mask") (roundrect_rratio 0.25) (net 4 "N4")))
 (gr_line (start 133 85) (end 141.514466 84.985534) (stroke (width 0.1) (type default)) (layer "Edge.Cuts"))
 (gr_arc (start 128 90) (mid 129.464466 86.464466) (end 133 85) (stroke (width 0.1) (type default)) (layer "Edge.Cuts"))
 (gr_line (start 146.514466 89.985534) (end 146.5 102.5) (stroke (width 0.1) (type default)) (layer "Edge.Cuts"))
 (gr_line (start 132.985534 107.014466) (end 142 107) (stroke (width 0.1) (type default)) (layer "Edge.Cuts"))
 (gr_arc (start 146.5 102.5) (mid 145.181981 105.681981) (end 142 107) (stroke (width 0.1) (type default)) (layer "Edge.Cuts"))
 (gr_arc (start 141.514466 84.985534) (mid 145.05 86.45) (end 146.514466 89.985534) (stroke (width 0.1) (type default)) (layer "Edge.Cuts"))
 (gr_line (start 128 90) (end 127.985534 102.014466) (stroke (width 0.1) (type default)) (layer "Edge.Cuts"))
 (gr_arc (start 132.985534 107.014466) (mid 129.45 105.55) (end 127.985534 102.014466) (stroke (width 0.1) (type default))
  (layer "Edge.Cuts"))
 (segment (start 130.7 97.8) (end 130 98.5) (width 0.25) (layer "F.Cu") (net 1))
 (segment (start 130.7 96.45) (end 130.7 97.8) (width 0.25) (layer "F.Cu") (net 1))
 (via (at 130 98.5) (size 0.8) (drill 0.4) (layers "F.Cu" "B.Cu") (free yes) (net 1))
 (segment (start 135.0875 96.5) (end 132.35 96.5) (width 0.25) (layer "F.Cu") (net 4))
 (segment (start 132.35 96.5) (end 132.3 96.45) (width 0.25) (layer "F.Cu") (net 4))
 (segment (start 136.9125 96.5) (end 136.9125 94.5875) (width 0.25) (layer "F.Cu") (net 3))
 (segment (start 137.5 94) (end 137.5 87.5) (width 0.25) (layer "F.Cu") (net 3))
 (segment (start 137.5 87.5) (end 137.705 87.295) (width 0.25) (layer "F.Cu") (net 3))
 (segment (start 137.705 87.295) (end 140.3 87.295) (width 0.25) (layer "F.Cu") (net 3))
 (segment (start 136.9125 94.5875) (end 137.5 94) (width 0.25) (layer "F.Cu") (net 3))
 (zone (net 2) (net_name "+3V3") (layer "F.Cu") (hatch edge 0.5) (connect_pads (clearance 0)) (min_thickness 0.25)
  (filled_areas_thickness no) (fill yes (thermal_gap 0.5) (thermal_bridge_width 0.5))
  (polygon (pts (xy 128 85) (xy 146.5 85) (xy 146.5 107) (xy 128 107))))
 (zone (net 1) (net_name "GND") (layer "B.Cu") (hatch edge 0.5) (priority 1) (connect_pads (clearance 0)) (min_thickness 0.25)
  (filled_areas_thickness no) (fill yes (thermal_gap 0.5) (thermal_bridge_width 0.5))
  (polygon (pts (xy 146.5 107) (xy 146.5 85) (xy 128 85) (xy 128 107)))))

